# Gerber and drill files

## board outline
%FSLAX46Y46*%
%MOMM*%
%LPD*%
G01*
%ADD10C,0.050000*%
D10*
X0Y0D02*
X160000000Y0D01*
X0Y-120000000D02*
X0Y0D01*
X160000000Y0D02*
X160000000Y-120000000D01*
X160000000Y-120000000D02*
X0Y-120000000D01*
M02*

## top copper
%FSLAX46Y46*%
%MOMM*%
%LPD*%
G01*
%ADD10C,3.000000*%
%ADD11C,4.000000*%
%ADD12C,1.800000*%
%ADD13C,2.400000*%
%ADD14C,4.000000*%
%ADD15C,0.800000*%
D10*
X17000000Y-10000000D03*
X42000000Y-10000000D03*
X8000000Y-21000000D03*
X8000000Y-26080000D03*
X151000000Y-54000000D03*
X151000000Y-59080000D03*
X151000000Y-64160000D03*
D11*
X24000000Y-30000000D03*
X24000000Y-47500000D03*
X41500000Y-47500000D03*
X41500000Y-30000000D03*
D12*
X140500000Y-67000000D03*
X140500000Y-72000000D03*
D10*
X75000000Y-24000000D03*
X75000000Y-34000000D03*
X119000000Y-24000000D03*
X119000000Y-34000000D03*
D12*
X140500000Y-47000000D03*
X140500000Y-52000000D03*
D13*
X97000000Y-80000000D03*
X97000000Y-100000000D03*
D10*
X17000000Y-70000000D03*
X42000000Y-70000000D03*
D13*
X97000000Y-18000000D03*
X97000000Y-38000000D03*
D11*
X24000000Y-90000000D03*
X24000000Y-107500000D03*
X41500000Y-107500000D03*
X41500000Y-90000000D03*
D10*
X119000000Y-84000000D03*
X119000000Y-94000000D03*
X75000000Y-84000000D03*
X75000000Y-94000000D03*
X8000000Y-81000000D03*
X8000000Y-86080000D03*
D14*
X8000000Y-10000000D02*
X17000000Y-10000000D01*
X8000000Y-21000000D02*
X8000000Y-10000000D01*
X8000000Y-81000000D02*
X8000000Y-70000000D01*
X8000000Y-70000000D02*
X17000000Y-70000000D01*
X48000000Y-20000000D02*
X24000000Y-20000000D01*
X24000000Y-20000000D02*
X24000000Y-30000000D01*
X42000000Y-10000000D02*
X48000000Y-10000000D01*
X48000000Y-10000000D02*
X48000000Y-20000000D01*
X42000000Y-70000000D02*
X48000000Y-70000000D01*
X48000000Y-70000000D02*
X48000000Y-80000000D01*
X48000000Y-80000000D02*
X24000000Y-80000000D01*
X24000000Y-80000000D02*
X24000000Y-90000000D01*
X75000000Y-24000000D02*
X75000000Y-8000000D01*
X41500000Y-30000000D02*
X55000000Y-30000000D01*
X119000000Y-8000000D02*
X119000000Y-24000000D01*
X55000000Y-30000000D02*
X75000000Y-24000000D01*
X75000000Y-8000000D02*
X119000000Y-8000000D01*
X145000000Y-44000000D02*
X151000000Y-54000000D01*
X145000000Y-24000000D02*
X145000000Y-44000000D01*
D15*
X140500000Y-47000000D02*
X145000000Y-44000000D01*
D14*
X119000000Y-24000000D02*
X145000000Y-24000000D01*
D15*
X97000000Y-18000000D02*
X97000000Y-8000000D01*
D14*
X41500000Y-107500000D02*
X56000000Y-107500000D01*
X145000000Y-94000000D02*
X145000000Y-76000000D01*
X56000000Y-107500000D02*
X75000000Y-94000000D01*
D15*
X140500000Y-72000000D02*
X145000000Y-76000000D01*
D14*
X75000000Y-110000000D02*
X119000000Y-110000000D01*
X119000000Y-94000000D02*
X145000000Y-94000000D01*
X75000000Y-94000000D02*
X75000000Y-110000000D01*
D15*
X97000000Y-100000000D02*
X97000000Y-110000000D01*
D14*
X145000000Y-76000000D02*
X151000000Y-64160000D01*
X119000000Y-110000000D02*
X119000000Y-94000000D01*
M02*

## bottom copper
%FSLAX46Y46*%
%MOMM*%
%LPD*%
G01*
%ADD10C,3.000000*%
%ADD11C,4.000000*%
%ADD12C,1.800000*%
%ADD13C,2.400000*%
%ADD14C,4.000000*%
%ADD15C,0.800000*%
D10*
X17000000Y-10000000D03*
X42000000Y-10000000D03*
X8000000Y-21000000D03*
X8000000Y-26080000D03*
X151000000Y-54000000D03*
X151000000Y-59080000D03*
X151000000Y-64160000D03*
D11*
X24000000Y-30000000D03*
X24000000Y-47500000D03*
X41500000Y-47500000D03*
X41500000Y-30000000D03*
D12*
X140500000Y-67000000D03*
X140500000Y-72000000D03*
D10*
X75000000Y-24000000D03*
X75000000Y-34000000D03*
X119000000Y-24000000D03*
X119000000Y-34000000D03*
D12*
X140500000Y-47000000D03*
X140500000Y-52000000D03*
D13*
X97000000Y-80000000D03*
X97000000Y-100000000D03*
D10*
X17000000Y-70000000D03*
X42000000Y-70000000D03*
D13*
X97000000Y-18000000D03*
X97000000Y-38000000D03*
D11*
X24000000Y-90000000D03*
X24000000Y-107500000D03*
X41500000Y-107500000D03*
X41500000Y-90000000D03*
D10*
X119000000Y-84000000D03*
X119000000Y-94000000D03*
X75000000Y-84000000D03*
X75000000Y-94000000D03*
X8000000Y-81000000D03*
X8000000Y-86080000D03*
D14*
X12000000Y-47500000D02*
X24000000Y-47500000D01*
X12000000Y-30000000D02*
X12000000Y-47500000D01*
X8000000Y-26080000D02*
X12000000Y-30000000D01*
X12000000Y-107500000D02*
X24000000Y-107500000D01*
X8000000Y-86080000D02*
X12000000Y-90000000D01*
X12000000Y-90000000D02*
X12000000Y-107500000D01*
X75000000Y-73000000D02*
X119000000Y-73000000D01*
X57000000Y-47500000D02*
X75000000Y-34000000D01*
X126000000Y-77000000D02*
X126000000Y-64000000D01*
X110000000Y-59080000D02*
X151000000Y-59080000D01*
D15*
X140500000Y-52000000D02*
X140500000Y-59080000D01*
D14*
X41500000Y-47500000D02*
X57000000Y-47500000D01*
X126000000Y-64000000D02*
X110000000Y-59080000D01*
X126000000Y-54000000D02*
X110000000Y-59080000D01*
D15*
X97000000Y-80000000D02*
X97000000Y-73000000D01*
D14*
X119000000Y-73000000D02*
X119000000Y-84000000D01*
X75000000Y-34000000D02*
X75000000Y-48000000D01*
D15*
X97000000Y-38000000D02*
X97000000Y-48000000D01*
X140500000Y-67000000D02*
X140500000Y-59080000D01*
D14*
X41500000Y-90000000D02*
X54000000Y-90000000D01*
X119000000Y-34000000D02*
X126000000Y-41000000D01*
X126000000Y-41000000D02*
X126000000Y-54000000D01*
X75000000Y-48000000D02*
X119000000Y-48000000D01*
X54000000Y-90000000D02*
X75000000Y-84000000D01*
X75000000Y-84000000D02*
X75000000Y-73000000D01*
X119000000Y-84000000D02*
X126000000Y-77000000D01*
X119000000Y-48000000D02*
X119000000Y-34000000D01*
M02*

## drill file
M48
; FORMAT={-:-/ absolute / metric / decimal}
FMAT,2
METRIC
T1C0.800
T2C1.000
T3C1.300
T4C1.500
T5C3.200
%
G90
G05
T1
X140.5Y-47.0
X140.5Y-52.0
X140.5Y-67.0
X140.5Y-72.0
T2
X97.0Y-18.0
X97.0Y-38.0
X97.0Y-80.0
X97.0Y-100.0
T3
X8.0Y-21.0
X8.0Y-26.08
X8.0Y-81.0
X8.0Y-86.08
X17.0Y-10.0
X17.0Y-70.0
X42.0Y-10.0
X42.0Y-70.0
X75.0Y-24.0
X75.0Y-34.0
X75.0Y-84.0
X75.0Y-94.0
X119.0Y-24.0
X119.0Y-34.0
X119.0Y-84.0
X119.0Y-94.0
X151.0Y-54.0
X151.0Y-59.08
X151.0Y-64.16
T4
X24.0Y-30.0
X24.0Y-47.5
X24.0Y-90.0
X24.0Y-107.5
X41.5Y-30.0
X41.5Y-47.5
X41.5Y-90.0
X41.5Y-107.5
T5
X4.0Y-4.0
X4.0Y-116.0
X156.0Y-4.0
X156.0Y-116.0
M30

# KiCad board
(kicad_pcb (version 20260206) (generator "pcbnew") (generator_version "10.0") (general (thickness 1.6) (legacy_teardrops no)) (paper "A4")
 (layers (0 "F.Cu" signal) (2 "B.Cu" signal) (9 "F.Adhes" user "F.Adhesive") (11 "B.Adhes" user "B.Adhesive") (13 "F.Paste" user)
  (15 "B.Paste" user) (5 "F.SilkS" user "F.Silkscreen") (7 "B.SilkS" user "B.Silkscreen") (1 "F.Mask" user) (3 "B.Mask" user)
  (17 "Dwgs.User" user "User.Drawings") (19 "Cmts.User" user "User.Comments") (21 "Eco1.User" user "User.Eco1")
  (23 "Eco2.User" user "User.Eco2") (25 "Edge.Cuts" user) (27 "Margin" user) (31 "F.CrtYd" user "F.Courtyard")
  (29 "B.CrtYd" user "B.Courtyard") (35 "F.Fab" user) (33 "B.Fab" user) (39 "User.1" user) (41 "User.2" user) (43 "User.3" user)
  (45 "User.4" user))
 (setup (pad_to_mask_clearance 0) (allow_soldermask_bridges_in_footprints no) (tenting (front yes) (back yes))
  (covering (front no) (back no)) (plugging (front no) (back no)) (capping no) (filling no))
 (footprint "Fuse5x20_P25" (layer "F.Cu") (at 17 10)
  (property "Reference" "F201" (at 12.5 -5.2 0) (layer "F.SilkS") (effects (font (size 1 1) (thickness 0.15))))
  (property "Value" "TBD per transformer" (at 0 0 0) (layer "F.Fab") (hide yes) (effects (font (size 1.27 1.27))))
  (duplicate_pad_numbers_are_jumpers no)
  (pad "1" thru_hole circle (at 0 0) (size 3 3) (drill 1.3) (layers "*.Cu" "*.Mask") (remove_unused_layers no) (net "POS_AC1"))
  (pad "2" thru_hole circle (at 25 0) (size 3 3) (drill 1.3) (layers "*.Cu" "*.Mask") (remove_unused_layers no) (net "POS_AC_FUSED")))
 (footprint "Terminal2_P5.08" (layer "F.Cu") (at 8 21 -90)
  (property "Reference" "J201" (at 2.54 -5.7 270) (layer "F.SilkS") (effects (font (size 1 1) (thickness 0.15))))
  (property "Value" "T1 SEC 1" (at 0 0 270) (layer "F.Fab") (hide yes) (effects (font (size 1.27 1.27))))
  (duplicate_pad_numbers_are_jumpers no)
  (pad "1" thru_hole circle (at 0 0 270) (size 3 3) (drill 1.3) (layers "*.Cu" "*.Mask") (remove_unused_layers no) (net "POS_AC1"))
  (pad "2" thru_hole circle (at 5.08 0 270) (size 3 3) (drill 1.3) (layers "*.Cu" "*.Mask") (remove_unused_layers no) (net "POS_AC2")))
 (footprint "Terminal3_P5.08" (layer "F.Cu") (at 151 54 -90)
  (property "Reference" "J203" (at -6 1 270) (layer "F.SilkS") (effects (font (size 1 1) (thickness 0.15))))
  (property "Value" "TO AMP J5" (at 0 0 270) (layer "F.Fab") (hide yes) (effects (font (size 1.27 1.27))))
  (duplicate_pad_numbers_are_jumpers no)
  (pad "1" thru_hole circle (at 0 0 270) (size 3 3) (drill 1.3) (layers "*.Cu" "*.Mask") (remove_unused_layers no) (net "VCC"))
  (pad "2" thru_hole circle (at 5.08 0 270) (size 3 3) (drill 1.3) (layers "*.Cu" "*.Mask") (remove_unused_layers no) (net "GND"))
  (pad "3" thru_hole circle (at 10.16 0 270) (size 3 3) (drill 1.3) (layers "*.Cu" "*.Mask") (remove_unused_layers no) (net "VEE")))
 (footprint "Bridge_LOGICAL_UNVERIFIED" (layer "F.Cu") (at 24 30)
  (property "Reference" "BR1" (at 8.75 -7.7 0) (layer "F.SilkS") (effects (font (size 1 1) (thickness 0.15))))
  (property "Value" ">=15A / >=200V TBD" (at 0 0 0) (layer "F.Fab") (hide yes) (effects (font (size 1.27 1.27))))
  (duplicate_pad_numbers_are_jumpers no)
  (pad "AC1" thru_hole circle (at 0 0) (size 4 4) (drill 1.5) (layers "*.Cu" "*.Mask") (remove_unused_layers no) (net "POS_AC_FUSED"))
  (pad "AC2" thru_hole circle (at 0 17.5) (size 4 4) (drill 1.5) (layers "*.Cu" "*.Mask") (remove_unused_layers no) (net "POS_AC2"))
  (pad "N" thru_hole circle (at 17.5 17.5) (size 4 4) (drill 1.5) (layers "*.Cu" "*.Mask") (remove_unused_layers no) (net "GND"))
  (pad "P" thru_hole circle (at 17.5 0) (size 4 4) (drill 1.5) (layers "*.Cu" "*.Mask") (remove_unused_layers no) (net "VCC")))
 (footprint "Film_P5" (layer "F.Cu") (at 140.5 67 -90)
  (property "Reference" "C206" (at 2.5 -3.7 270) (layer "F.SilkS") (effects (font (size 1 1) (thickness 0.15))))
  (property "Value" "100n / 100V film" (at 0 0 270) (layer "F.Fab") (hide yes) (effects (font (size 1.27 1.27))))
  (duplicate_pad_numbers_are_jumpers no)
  (pad "1" thru_hole circle (at 0 0 270) (size 1.8 1.8) (drill 0.8) (layers "*.Cu" "*.Mask") (remove_unused_layers no) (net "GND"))
  (pad "2" thru_hole circle (at 5 0 270) (size 1.8 1.8) (drill 0.8) (layers "*.Cu" "*.Mask") (remove_unused_layers no) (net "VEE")))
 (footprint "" (layer "F.Cu") (at 156 116)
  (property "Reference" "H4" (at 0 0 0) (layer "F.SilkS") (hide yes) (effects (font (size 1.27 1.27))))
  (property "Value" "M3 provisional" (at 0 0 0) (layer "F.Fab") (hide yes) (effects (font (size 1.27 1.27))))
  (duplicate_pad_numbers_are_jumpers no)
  (pad "" np_thru_hole circle (at 0 0) (size 3.2 3.2) (drill 3.2) (layers "*.Cu" "*.Mask")))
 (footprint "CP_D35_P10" (layer "F.Cu") (at 75 24 -90)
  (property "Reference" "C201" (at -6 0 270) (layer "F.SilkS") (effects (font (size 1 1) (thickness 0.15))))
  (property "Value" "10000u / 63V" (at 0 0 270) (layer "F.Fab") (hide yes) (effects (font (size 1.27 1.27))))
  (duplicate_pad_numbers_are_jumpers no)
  (pad "1" thru_hole circle (at 0 0 270) (size 3 3) (drill 1.3) (layers "*.Cu" "*.Mask") (remove_unused_layers no) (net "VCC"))
  (pad "2" thru_hole circle (at 10 0 270) (size 3 3) (drill 1.3) (layers "*.Cu" "*.Mask") (remove_unused_layers no) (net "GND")))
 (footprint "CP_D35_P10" (layer "F.Cu") (at 119 24 -90)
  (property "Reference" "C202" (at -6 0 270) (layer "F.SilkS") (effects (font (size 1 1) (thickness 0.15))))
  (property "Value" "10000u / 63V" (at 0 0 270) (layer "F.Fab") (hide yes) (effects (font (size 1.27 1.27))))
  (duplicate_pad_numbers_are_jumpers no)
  (pad "1" thru_hole circle (at 0 0 270) (size 3 3) (drill 1.3) (layers "*.Cu" "*.Mask") (remove_unused_layers no) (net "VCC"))
  (pad "2" thru_hole circle (at 10 0 270) (size 3 3) (drill 1.3) (layers "*.Cu" "*.Mask") (remove_unused_layers no) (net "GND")))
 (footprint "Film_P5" (layer "F.Cu") (at 140.5 47 -90)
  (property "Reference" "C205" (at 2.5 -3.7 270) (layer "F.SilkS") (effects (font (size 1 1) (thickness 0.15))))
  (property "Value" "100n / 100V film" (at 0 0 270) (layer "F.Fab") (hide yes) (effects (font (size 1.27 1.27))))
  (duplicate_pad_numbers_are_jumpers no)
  (pad "1" thru_hole circle (at 0 0 270) (size 1.8 1.8) (drill 0.8) (layers "*.Cu" "*.Mask") (remove_unused_layers no) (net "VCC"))
  (pad "2" thru_hole circle (at 5 0 270) (size 1.8 1.8) (drill 0.8) (layers "*.Cu" "*.Mask") (remove_unused_layers no) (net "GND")))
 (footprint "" (layer "F.Cu") (at 4 4)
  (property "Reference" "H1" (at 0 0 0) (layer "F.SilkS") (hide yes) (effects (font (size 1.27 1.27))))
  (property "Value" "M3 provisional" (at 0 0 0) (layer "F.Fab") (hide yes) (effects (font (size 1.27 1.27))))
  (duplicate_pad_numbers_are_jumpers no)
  (pad "" np_thru_hole circle (at 0 0) (size 3.2 3.2) (drill 3.2) (layers "*.Cu" "*.Mask")))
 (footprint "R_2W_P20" (layer "F.Cu") (at 97 80 -90)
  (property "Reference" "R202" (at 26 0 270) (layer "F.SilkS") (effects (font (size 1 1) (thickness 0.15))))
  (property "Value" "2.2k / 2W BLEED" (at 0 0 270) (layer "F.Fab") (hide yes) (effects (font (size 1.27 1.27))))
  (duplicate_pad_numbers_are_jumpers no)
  (pad "1" thru_hole circle (at 0 0 270) (size 2.4 2.4) (drill 1) (layers "*.Cu" "*.Mask") (remove_unused_layers no) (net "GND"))
  (pad "2" thru_hole circle (at 20 0 270) (size 2.4 2.4) (drill 1) (layers "*.Cu" "*.Mask") (remove_unused_layers no) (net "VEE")))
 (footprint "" (layer "F.Cu") (at 156 4)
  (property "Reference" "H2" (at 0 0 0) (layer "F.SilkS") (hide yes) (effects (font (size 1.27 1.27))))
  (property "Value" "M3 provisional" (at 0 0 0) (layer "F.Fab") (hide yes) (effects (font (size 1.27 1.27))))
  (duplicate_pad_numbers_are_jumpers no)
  (pad "" np_thru_hole circle (at 0 0) (size 3.2 3.2) (drill 3.2) (layers "*.Cu" "*.Mask")))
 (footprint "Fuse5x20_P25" (layer "F.Cu") (at 17 70)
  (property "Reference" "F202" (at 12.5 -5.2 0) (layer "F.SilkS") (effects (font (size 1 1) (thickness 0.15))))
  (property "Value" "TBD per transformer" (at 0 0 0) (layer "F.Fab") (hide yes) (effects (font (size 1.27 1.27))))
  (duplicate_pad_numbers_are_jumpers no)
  (pad "1" thru_hole circle (at 0 0) (size 3 3) (drill 1.3) (layers "*.Cu" "*.Mask") (remove_unused_layers no) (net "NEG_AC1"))
  (pad "2" thru_hole circle (at 25 0) (size 3 3) (drill 1.3) (layers "*.Cu" "*.Mask") (remove_unused_layers no) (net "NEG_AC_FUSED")))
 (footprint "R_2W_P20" (layer "F.Cu") (at 97 18 -90)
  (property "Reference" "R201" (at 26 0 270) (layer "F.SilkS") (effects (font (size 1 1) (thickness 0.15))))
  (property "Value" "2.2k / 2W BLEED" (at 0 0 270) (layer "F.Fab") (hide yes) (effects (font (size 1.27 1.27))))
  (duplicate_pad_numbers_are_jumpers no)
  (pad "1" thru_hole circle (at 0 0 270) (size 2.4 2.4) (drill 1) (layers "*.Cu" "*.Mask") (remove_unused_layers no) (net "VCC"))
  (pad "2" thru_hole circle (at 20 0 270) (size 2.4 2.4) (drill 1) (layers "*.Cu" "*.Mask") (remove_unused_layers no) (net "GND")))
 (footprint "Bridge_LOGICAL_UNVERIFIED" (layer "F.Cu") (at 24 90)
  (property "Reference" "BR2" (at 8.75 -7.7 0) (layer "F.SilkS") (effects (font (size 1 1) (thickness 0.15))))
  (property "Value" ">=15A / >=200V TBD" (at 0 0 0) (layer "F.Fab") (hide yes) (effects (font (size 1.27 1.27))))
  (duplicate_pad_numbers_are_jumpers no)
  (pad "AC1" thru_hole circle (at 0 0) (size 4 4) (drill 1.5) (layers "*.Cu" "*.Mask") (remove_unused_layers no) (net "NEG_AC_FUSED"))
  (pad "AC2" thru_hole circle (at 0 17.5) (size 4 4) (drill 1.5) (layers "*.Cu" "*.Mask") (remove_unused_layers no) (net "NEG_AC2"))
  (pad "N" thru_hole circle (at 17.5 17.5) (size 4 4) (drill 1.5) (layers "*.Cu" "*.Mask") (remove_unused_layers no) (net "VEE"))
  (pad "P" thru_hole circle (at 17.5 0) (size 4 4) (drill 1.5) (layers "*.Cu" "*.Mask") (remove_unused_layers no) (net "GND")))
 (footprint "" (layer "F.Cu") (at 4 116)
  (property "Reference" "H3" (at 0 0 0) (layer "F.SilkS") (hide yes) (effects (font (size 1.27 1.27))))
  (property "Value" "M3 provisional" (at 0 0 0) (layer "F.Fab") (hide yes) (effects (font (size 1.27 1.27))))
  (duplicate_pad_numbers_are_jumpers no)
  (pad "" np_thru_hole circle (at 0 0) (size 3.2 3.2) (drill 3.2) (layers "*.Cu" "*.Mask")))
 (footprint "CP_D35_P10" (layer "F.Cu") (at 119 84 -90)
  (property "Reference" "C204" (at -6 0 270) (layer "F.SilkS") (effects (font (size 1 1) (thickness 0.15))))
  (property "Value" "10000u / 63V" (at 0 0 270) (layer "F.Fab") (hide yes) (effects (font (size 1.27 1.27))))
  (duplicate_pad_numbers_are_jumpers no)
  (pad "1" thru_hole circle (at 0 0 270) (size 3 3) (drill 1.3) (layers "*.Cu" "*.Mask") (remove_unused_layers no) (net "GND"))
  (pad "2" thru_hole circle (at 10 0 270) (size 3 3) (drill 1.3) (layers "*.Cu" "*.Mask") (remove_unused_layers no) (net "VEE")))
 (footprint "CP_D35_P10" (layer "F.Cu") (at 75 84 -90)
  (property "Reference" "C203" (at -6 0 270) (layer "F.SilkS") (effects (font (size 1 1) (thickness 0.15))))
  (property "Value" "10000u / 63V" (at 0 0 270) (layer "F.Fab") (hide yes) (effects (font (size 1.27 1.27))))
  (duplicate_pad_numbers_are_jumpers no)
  (pad "1" thru_hole circle (at 0 0 270) (size 3 3) (drill 1.3) (layers "*.Cu" "*.Mask") (remove_unused_layers no) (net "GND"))
  (pad "2" thru_hole circle (at 10 0 270) (size 3 3) (drill 1.3) (layers "*.Cu" "*.Mask") (remove_unused_layers no) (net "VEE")))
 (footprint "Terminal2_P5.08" (layer "F.Cu") (at 8 81 -90)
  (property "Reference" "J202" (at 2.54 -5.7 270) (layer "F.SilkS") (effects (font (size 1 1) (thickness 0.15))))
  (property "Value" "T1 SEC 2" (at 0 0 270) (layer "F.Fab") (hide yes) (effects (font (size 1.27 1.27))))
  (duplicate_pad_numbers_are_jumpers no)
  (pad "1" thru_hole circle (at 0 0 270) (size 3 3) (drill 1.3) (layers "*.Cu" "*.Mask") (remove_unused_layers no) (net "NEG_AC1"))
  (pad "2" thru_hole circle (at 5.08 0 270) (size 3 3) (drill 1.3) (layers "*.Cu" "*.Mask") (remove_unused_layers no) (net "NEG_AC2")))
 (gr_line (start 0 0) (end 160 0) (stroke (width 0.05) (type default)) (layer "Edge.Cuts"))
 (gr_line (start 0 120) (end 0 0) (stroke (width 0.05) (type default)) (layer "Edge.Cuts"))
 (gr_line (start 160 0) (end 160 120) (stroke (width 0.05) (type default)) (layer "Edge.Cuts"))
 (gr_line (start 160 120) (end 0 120) (stroke (width 0.05) (type default)) (layer "Edge.Cuts"))
 (segment (start 8 10) (end 17 10) (width 4) (layer "F.Cu") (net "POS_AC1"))
 (segment (start 8 21) (end 8 10) (width 4) (layer "F.Cu") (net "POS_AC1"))
 (segment (start 12 47.5) (end 24 47.5) (width 4) (layer "B.Cu") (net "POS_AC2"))
 (segment (start 12 30) (end 12 47.5) (width 4) (layer "B.Cu") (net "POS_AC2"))
 (segment (start 8 26.08) (end 12 30) (width 4) (layer "B.Cu") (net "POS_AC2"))
 (segment (start 8 81) (end 8 70) (width 4) (layer "F.Cu") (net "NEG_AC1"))
 (segment (start 8 70) (end 17 70) (width 4) (layer "F.Cu") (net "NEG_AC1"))
 (segment (start 12 107.5) (end 24 107.5) (width 4) (layer "B.Cu") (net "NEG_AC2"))
 (segment (start 8 86.08) (end 12 90) (width 4) (layer "B.Cu") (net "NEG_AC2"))
 (segment (start 12 90) (end 12 107.5) (width 4) (layer "B.Cu") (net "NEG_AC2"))
 (segment (start 48 20) (end 24 20) (width 4) (layer "F.Cu") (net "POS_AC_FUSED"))
 (segment (start 24 20) (end 24 30) (width 4) (layer "F.Cu") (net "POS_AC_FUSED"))
 (segment (start 42 10) (end 48 10) (width 4) (layer "F.Cu") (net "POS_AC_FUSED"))
 (segment (start 48 10) (end 48 20) (width 4) (layer "F.Cu") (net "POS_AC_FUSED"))
 (segment (start 42 70) (end 48 70) (width 4) (layer "F.Cu") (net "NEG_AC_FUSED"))
 (segment (start 48 70) (end 48 80) (width 4) (layer "F.Cu") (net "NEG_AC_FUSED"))
 (segment (start 48 80) (end 24 80) (width 4) (layer "F.Cu") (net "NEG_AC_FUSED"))
 (segment (start 24 80) (end 24 90) (width 4) (layer "F.Cu") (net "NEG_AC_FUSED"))
 (segment (start 75 73) (end 119 73) (width 4) (layer "B.Cu") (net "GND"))
 (segment (start 57 47.5) (end 75 34) (width 4) (layer "B.Cu") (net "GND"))
 (segment (start 126 77) (end 126 64) (width 4) (layer "B.Cu") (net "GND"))
 (segment (start 110 59.08) (end 151 59.08) (width 4) (layer "B.Cu") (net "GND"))
 (segment (start 140.5 52) (end 140.5 59.08) (width 0.8) (layer "B.Cu") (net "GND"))
 (segment (start 41.5 47.5) (end 57 47.5) (width 4) (layer "B.Cu") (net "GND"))
 (segment (start 126 64) (end 110 59.08) (width 4) (layer "B.Cu") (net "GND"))
 (segment (start 126 54) (end 110 59.08) (width 4) (layer "B.Cu") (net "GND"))
 (segment (start 97 80) (end 97 73) (width 0.8) (layer "B.Cu") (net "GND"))
 (segment (start 119 73) (end 119 84) (width 4) (layer "B.Cu") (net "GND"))
 (segment (start 75 34) (end 75 48) (width 4) (layer "B.Cu") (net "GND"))
 (segment (start 97 38) (end 97 48) (width 0.8) (layer "B.Cu") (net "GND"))
 (segment (start 140.5 67) (end 140.5 59.08) (width 0.8) (layer "B.Cu") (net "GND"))
 (segment (start 41.5 90) (end 54 90) (width 4) (layer "B.Cu") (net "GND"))
 (segment (start 119 34) (end 126 41) (width 4) (layer "B.Cu") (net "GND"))
 (segment (start 126 41) (end 126 54) (width 4) (layer "B.Cu") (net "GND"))
 (segment (start 75 48) (end 119 48) (width 4) (layer "B.Cu") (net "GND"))
 (segment (start 54 90) (end 75 84) (width 4) (layer "B.Cu") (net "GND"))
 (segment (start 75 84) (end 75 73) (width 4) (layer "B.Cu") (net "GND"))
 (segment (start 119 84) (end 126 77) (width 4) (layer "B.Cu") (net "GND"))
 (segment (start 119 48) (end 119 34) (width 4) (layer "B.Cu") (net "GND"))
 (segment (start 75 24) (end 75 8) (width 4) (layer "F.Cu") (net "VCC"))
 (segment (start 41.5 30) (end 55 30) (width 4) (layer "F.Cu") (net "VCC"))
 (segment (start 119 8) (end 119 24) (width 4) (layer "F.Cu") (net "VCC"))
 (segment (start 55 30) (end 75 24) (width 4) (layer "F.Cu") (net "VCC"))
 (segment (start 75 8) (end 119 8) (width 4) (layer "F.Cu") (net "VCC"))
 (segment (start 145 44) (end 151 54) (width 4) (layer "F.Cu") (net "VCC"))
 (segment (start 145 24) (end 145 44) (width 4) (layer "F.Cu") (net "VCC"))
 (segment (start 140.5 47) (end 145 44) (width 0.8) (layer "F.Cu") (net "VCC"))
 (segment (start 119 24) (end 145 24) (width 4) (layer "F.Cu") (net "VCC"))
 (segment (start 97 18) (end 97 8) (width 0.8) (layer "F.Cu") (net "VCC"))
 (segment (start 41.5 107.5) (end 56 107.5) (width 4) (layer "F.Cu") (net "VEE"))
 (segment (start 145 94) (end 145 76) (width 4) (layer "F.Cu") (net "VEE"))
 (segment (start 56 107.5) (end 75 94) (width 4) (layer "F.Cu") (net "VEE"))
 (segment (start 140.5 72) (end 145 76) (width 0.8) (layer "F.Cu") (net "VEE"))
 (segment (start 75 110) (end 119 110) (width 4) (layer "F.Cu") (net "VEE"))
 (segment (start 119 94) (end 145 94) (width 4) (layer "F.Cu") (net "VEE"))
 (segment (start 75 94) (end 75 110) (width 4) (layer "F.Cu") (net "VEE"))
 (segment (start 97 100) (end 97 110) (width 0.8) (layer "F.Cu") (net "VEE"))
 (segment (start 145 76) (end 151 64.16) (width 4) (layer "F.Cu") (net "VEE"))
 (segment (start 119 110) (end 119 94) (width 4) (layer "F.Cu") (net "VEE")))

